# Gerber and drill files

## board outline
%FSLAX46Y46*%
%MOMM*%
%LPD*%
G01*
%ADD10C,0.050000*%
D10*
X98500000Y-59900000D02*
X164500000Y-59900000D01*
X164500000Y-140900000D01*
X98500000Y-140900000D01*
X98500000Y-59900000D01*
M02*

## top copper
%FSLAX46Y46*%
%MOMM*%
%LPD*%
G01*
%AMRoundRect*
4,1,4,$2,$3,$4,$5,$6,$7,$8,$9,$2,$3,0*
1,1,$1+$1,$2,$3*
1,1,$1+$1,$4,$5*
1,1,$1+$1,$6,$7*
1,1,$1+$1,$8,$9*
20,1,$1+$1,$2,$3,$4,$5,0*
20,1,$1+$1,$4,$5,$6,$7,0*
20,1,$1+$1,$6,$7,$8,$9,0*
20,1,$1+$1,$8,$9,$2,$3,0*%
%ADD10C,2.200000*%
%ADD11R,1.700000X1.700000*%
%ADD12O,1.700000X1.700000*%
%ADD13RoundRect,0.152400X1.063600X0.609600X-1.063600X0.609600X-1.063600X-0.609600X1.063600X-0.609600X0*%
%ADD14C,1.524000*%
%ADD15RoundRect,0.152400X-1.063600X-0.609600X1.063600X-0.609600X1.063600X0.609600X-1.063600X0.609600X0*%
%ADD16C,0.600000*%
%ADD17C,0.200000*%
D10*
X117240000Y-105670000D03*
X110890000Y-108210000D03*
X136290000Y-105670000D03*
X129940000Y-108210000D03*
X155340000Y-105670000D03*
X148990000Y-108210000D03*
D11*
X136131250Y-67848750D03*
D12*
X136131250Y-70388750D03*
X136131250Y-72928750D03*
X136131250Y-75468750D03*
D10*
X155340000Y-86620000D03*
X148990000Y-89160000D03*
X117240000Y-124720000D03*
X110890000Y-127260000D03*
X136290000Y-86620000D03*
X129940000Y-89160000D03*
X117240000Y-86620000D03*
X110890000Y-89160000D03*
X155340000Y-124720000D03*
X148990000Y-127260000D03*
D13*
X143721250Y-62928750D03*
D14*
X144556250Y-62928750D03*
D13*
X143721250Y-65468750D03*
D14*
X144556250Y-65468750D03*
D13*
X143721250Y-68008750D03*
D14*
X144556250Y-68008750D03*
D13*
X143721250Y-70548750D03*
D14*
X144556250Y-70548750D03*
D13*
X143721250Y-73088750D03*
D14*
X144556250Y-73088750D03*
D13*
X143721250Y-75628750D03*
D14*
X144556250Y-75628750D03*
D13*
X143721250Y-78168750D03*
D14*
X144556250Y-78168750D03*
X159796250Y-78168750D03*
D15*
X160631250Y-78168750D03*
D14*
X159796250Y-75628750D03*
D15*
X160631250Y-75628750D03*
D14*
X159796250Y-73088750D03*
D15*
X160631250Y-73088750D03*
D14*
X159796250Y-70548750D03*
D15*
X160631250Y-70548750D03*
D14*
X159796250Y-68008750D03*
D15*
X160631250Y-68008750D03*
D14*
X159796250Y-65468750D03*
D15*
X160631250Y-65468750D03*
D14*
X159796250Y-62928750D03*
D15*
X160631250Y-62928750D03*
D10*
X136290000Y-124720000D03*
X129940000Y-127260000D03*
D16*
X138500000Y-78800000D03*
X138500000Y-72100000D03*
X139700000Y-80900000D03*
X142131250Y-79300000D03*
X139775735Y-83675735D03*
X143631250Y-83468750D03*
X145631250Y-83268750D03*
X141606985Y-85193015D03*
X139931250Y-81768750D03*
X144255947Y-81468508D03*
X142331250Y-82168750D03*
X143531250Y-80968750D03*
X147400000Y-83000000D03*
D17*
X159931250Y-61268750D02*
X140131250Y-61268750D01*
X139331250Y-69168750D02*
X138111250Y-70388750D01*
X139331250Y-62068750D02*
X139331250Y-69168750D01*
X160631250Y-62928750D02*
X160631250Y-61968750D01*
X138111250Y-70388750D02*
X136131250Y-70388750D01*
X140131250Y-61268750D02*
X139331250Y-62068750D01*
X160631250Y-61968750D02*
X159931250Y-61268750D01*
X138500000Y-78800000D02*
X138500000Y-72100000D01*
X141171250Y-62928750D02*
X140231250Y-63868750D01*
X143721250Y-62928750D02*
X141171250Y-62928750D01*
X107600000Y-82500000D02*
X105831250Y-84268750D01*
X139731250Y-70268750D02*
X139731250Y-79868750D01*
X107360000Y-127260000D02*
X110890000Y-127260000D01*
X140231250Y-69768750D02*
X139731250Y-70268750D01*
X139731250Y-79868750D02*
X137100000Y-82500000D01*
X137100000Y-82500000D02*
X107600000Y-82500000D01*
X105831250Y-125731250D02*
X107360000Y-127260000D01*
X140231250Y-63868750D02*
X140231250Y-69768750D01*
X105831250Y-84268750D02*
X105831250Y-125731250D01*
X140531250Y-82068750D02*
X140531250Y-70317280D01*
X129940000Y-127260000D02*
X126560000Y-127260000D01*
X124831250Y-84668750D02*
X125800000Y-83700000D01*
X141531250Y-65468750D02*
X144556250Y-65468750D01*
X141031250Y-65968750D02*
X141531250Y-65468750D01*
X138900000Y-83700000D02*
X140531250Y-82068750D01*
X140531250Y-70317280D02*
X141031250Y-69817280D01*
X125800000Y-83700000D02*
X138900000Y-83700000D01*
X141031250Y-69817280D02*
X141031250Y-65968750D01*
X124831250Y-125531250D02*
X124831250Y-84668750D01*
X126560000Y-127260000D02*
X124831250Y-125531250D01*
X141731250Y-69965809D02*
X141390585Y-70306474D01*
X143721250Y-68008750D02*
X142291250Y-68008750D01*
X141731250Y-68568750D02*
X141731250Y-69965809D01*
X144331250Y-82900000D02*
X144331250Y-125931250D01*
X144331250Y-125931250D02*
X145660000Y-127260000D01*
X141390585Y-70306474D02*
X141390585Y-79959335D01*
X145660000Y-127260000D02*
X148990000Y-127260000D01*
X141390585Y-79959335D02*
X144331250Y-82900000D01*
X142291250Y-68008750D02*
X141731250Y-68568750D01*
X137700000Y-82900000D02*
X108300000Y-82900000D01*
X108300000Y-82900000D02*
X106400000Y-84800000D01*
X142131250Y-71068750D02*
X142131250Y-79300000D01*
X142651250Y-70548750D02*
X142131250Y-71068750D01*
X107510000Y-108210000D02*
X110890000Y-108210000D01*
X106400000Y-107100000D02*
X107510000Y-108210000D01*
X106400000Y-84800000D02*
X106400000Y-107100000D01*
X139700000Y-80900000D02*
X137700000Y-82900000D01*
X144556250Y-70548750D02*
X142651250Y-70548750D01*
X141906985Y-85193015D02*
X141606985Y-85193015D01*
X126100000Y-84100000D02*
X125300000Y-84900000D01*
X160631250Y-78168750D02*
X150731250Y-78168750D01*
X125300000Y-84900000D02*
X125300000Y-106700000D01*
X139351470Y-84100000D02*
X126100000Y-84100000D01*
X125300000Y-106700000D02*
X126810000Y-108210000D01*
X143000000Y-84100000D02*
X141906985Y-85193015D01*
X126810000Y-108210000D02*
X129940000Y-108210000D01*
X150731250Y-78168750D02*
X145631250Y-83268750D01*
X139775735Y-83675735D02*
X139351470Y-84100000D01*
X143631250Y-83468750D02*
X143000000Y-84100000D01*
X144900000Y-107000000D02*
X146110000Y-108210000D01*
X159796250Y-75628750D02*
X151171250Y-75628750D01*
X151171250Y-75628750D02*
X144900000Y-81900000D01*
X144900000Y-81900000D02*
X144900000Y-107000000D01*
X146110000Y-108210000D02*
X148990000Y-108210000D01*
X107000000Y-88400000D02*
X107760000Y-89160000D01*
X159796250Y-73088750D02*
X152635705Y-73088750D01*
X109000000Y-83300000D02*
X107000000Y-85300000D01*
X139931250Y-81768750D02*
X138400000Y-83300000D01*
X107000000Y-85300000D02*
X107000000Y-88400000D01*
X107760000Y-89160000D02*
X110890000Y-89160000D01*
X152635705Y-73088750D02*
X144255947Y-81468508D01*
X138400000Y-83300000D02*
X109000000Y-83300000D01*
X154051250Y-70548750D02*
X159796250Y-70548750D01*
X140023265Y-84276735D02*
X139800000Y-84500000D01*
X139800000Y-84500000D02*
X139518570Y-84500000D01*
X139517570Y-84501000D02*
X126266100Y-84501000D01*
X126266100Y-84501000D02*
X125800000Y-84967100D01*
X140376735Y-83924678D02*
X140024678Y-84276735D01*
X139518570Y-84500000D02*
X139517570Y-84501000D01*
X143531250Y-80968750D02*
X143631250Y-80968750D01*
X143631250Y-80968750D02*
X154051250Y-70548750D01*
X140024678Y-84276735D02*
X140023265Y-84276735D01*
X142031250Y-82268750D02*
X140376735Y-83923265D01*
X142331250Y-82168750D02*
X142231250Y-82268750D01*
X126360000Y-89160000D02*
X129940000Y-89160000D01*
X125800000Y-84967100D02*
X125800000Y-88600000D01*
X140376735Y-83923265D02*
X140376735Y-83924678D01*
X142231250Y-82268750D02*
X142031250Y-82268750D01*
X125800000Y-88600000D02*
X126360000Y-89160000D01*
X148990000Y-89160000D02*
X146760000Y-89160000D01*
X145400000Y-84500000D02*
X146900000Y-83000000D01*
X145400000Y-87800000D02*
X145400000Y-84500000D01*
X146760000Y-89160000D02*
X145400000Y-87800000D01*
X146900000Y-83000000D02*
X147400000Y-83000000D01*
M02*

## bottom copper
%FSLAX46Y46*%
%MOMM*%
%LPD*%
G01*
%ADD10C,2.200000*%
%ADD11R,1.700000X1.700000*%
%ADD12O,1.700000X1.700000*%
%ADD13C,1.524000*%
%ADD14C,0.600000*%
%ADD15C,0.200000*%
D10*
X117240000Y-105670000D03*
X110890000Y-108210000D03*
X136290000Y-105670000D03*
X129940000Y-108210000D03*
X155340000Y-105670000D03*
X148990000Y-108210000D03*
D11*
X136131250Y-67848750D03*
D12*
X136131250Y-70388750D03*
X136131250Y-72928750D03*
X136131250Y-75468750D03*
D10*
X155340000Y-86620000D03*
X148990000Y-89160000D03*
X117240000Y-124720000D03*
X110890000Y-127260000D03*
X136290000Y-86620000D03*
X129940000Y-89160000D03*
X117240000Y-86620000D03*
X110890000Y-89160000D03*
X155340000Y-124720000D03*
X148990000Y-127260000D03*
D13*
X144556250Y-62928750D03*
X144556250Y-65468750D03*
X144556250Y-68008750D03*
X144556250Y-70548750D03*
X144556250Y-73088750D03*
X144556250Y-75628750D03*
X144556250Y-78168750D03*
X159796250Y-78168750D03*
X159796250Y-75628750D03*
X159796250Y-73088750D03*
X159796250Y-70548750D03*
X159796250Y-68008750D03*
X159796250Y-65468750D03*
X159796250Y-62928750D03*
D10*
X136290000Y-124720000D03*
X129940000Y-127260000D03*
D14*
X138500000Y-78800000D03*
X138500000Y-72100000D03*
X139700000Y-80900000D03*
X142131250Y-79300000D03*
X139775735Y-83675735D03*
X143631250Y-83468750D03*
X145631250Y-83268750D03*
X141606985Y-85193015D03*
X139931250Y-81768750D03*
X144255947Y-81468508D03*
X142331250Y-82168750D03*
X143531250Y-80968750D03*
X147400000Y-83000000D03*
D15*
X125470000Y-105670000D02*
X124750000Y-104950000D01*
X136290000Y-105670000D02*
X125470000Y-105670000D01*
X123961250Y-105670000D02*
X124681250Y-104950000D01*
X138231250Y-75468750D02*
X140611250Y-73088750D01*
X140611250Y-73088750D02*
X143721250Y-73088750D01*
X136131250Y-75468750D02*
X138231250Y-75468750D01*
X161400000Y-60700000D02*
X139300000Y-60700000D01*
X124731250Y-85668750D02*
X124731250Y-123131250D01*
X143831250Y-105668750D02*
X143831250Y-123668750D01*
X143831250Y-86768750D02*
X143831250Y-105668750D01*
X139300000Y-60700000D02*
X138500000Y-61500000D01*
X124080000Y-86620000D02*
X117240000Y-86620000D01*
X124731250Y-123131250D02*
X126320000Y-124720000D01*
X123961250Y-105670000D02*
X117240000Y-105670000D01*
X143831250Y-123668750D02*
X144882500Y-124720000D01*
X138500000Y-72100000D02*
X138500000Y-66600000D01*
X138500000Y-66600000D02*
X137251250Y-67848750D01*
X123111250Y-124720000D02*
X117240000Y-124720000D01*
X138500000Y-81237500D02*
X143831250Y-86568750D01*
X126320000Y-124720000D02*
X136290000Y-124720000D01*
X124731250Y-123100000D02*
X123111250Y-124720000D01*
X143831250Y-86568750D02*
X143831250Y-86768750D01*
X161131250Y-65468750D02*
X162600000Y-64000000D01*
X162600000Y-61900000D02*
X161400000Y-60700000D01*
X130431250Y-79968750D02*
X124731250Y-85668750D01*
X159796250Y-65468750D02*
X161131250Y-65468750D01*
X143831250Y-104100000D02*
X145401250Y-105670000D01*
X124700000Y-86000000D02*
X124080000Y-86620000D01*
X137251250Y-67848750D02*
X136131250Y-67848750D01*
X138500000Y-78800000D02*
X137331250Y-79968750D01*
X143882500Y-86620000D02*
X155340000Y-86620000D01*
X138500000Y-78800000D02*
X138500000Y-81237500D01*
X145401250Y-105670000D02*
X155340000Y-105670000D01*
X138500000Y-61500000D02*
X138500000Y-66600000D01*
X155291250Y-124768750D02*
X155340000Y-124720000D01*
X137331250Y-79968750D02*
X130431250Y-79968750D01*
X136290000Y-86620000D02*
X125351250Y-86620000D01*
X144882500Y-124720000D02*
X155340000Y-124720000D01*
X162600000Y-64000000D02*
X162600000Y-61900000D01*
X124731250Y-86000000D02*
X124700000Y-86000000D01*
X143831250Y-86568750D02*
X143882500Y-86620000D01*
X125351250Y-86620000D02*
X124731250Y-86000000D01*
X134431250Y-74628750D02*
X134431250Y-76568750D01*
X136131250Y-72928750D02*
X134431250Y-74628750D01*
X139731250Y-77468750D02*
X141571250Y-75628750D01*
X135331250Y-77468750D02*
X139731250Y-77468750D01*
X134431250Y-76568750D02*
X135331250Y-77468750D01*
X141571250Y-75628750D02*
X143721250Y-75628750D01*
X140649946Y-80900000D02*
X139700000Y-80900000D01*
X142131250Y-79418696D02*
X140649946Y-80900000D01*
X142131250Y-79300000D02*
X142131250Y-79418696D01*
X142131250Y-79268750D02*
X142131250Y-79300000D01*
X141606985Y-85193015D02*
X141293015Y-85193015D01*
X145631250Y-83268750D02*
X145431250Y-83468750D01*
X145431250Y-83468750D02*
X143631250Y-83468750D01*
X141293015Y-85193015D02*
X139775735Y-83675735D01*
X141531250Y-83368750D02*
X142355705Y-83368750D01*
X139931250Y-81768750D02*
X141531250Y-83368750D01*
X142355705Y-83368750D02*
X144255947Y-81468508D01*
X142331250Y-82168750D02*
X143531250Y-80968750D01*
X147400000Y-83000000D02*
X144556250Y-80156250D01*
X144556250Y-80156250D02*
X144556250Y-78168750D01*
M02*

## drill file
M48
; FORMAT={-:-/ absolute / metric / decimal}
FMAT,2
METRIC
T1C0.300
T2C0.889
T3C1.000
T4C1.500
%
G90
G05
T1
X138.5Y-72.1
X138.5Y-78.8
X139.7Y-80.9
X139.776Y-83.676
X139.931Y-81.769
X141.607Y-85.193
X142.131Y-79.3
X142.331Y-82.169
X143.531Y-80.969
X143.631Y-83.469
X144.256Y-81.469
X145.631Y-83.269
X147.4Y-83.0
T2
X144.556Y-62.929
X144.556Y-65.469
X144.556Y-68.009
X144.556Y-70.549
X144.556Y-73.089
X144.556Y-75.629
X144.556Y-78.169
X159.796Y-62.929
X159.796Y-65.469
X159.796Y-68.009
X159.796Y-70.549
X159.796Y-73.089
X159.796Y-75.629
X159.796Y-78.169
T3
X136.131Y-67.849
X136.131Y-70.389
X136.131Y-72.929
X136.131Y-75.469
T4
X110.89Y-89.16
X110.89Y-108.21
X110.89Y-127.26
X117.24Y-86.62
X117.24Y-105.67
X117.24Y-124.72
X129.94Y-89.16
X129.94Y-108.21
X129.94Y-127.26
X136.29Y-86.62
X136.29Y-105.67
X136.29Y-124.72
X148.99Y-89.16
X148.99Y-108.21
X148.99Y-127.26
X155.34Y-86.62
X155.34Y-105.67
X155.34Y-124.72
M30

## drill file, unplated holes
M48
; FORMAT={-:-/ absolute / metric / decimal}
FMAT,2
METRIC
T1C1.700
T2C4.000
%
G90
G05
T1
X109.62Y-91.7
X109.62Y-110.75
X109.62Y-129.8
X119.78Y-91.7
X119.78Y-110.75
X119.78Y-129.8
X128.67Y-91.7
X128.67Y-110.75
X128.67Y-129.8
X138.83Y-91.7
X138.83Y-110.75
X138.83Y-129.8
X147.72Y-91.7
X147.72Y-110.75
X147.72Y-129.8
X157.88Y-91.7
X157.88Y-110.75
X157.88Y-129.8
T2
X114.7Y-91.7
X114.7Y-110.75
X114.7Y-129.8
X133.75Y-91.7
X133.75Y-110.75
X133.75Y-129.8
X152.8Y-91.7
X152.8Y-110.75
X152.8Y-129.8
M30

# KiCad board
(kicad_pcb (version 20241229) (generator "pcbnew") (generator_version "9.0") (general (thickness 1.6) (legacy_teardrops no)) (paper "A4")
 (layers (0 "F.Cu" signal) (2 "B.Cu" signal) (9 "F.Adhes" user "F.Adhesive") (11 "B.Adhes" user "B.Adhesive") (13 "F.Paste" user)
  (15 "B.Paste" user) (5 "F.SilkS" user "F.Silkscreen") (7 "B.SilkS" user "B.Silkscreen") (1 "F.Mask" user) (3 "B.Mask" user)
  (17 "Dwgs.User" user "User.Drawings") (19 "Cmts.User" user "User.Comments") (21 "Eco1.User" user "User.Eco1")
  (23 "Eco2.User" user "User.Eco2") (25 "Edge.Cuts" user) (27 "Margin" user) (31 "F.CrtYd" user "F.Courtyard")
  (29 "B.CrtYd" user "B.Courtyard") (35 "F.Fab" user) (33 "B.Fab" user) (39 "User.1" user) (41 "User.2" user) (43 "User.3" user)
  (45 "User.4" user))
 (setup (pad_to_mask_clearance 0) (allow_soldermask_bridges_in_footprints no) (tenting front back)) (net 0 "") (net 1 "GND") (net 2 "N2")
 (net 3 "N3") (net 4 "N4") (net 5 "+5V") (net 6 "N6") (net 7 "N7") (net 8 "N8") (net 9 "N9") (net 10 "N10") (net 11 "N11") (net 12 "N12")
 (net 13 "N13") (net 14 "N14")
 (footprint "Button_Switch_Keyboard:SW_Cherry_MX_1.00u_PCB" (layer "F.Cu") (at 117.24 105.67)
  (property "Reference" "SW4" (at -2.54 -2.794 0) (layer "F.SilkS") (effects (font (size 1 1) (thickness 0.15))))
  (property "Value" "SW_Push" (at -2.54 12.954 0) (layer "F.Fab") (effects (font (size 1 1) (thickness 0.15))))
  (pad "" np_thru_hole circle (at -7.62 5.08) (size 1.7 1.7) (drill 1.7) (layers "*.Cu" "*.Mask"))
  (pad "" np_thru_hole circle (at -2.54 5.08) (size 4 4) (drill 4) (layers "*.Cu" "*.Mask"))
  (pad "" np_thru_hole circle (at 2.54 5.08) (size 1.7 1.7) (drill 1.7) (layers "*.Cu" "*.Mask"))
  (pad "1" thru_hole circle (at 0 0) (size 2.2 2.2) (drill 1.5) (layers "*.Cu" "*.Mask") (remove_unused_layers no) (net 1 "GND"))
  (pad "2" thru_hole circle (at -6.35 2.54) (size 2.2 2.2) (drill 1.5) (layers "*.Cu" "*.Mask") (remove_unused_layers no) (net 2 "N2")))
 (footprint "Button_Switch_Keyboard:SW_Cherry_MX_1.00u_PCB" (layer "F.Cu") (at 136.29 105.67)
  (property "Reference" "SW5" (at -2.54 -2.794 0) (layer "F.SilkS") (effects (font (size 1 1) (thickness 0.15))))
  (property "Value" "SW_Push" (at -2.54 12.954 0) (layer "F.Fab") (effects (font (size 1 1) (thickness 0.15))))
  (pad "" np_thru_hole circle (at -7.62 5.08) (size 1.7 1.7) (drill 1.7) (layers "*.Cu" "*.Mask"))
  (pad "" np_thru_hole circle (at -2.54 5.08) (size 4 4) (drill 4) (layers "*.Cu" "*.Mask"))
  (pad "" np_thru_hole circle (at 2.54 5.08) (size 1.7 1.7) (drill 1.7) (layers "*.Cu" "*.Mask"))
  (pad "1" thru_hole circle (at 0 0) (size 2.2 2.2) (drill 1.5) (layers "*.Cu" "*.Mask") (remove_unused_layers no) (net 1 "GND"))
  (pad "2" thru_hole circle (at -6.35 2.54) (size 2.2 2.2) (drill 1.5) (layers "*.Cu" "*.Mask") (remove_unused_layers no) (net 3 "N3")))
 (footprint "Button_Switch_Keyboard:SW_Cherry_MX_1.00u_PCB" (layer "F.Cu") (at 155.34 105.67)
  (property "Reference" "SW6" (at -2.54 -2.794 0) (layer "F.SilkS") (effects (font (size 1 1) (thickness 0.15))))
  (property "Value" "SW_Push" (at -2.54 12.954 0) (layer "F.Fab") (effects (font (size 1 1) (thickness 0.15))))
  (pad "" np_thru_hole circle (at -7.62 5.08) (size 1.7 1.7) (drill 1.7) (layers "*.Cu" "*.Mask"))
  (pad "" np_thru_hole circle (at -2.54 5.08) (size 4 4) (drill 4) (layers "*.Cu" "*.Mask"))
  (pad "" np_thru_hole circle (at 2.54 5.08) (size 1.7 1.7) (drill 1.7) (layers "*.Cu" "*.Mask"))
  (pad "1" thru_hole circle (at 0 0) (size 2.2 2.2) (drill 1.5) (layers "*.Cu" "*.Mask") (remove_unused_layers no) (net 1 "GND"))
  (pad "2" thru_hole circle (at -6.35 2.54) (size 2.2 2.2) (drill 1.5) (layers "*.Cu" "*.Mask") (remove_unused_layers no) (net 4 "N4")))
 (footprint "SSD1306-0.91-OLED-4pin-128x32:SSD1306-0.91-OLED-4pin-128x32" (layer "F.Cu") (at 99.63125 65.65875)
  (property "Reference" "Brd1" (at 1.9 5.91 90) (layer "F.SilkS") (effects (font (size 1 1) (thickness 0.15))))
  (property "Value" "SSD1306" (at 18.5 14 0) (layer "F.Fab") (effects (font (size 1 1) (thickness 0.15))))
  (pad "1" thru_hole rect (at 36.5 2.19) (size 1.7 1.7) (drill 1) (layers "*.Cu" "*.Mask") (remove_unused_layers no) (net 1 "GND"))
  (pad "2" thru_hole oval (at 36.5 4.73) (size 1.7 1.7) (drill 1) (layers "*.Cu" "*.Mask") (remove_unused_layers no) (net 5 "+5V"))
  (pad "3" thru_hole oval (at 36.5 7.27) (size 1.7 1.7) (drill 1) (layers "*.Cu" "*.Mask") (remove_unused_layers no) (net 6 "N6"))
  (pad "4" thru_hole oval (at 36.5 9.81) (size 1.7 1.7) (drill 1) (layers "*.Cu" "*.Mask") (remove_unused_layers no) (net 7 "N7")))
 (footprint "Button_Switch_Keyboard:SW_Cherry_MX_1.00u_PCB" (layer "F.Cu") (at 155.34 86.62)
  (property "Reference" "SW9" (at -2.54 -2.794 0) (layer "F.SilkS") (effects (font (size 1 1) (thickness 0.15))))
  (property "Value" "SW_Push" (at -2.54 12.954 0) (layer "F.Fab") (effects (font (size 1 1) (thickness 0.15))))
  (pad "" np_thru_hole circle (at -7.62 5.08) (size 1.7 1.7) (drill 1.7) (layers "*.Cu" "*.Mask"))
  (pad "" np_thru_hole circle (at -2.54 5.08) (size 4 4) (drill 4) (layers "*.Cu" "*.Mask"))
  (pad "" np_thru_hole circle (at 2.54 5.08) (size 1.7 1.7) (drill 1.7) (layers "*.Cu" "*.Mask"))
  (pad "1" thru_hole circle (at 0 0) (size 2.2 2.2) (drill 1.5) (layers "*.Cu" "*.Mask") (remove_unused_layers no) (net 1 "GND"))
  (pad "2" thru_hole circle (at -6.35 2.54) (size 2.2 2.2) (drill 1.5) (layers "*.Cu" "*.Mask") (remove_unused_layers no) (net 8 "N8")))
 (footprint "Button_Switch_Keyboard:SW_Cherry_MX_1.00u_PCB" (layer "F.Cu") (at 117.24 124.72)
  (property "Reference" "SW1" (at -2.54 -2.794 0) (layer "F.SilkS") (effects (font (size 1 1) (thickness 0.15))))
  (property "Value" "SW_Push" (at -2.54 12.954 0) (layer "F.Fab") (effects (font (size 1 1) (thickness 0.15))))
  (pad "" np_thru_hole circle (at -7.62 5.08) (size 1.7 1.7) (drill 1.7) (layers "*.Cu" "*.Mask"))
  (pad "" np_thru_hole circle (at -2.54 5.08) (size 4 4) (drill 4) (layers "*.Cu" "*.Mask"))
  (pad "" np_thru_hole circle (at 2.54 5.08) (size 1.7 1.7) (drill 1.7) (layers "*.Cu" "*.Mask"))
  (pad "1" thru_hole circle (at 0 0) (size 2.2 2.2) (drill 1.5) (layers "*.Cu" "*.Mask") (remove_unused_layers no) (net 1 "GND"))
  (pad "2" thru_hole circle (at -6.35 2.54) (size 2.2 2.2) (drill 1.5) (layers "*.Cu" "*.Mask") (remove_unused_layers no) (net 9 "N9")))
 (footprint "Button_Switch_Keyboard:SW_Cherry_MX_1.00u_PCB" (layer "F.Cu") (at 136.29 86.62)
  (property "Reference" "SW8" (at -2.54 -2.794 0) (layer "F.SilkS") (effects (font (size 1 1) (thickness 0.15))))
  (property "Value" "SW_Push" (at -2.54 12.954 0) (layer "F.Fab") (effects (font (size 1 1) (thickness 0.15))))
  (pad "" np_thru_hole circle (at -7.62 5.08) (size 1.7 1.7) (drill 1.7) (layers "*.Cu" "*.Mask"))
  (pad "" np_thru_hole circle (at -2.54 5.08) (size 4 4) (drill 4) (layers "*.Cu" "*.Mask"))
  (pad "" np_thru_hole circle (at 2.54 5.08) (size 1.7 1.7) (drill 1.7) (layers "*.Cu" "*.Mask"))
  (pad "1" thru_hole circle (at 0 0) (size 2.2 2.2) (drill 1.5) (layers "*.Cu" "*.Mask") (remove_unused_layers no) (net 1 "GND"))
  (pad "2" thru_hole circle (at -6.35 2.54) (size 2.2 2.2) (drill 1.5) (layers "*.Cu" "*.Mask") (remove_unused_layers no) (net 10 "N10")))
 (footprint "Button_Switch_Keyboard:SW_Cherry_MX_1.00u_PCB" (layer "F.Cu") (at 117.24 86.62)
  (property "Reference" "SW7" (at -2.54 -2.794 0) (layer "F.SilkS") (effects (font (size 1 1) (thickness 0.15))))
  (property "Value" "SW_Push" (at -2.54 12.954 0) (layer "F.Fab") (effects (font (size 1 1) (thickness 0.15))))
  (pad "" np_thru_hole circle (at -7.62 5.08) (size 1.7 1.7) (drill 1.7) (layers "*.Cu" "*.Mask"))
  (pad "" np_thru_hole circle (at -2.54 5.08) (size 4 4) (drill 4) (layers "*.Cu" "*.Mask"))
  (pad "" np_thru_hole circle (at 2.54 5.08) (size 1.7 1.7) (drill 1.7) (layers "*.Cu" "*.Mask"))
  (pad "1" thru_hole circle (at 0 0) (size 2.2 2.2) (drill 1.5) (layers "*.Cu" "*.Mask") (remove_unused_layers no) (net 1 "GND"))
  (pad "2" thru_hole circle (at -6.35 2.54) (size 2.2 2.2) (drill 1.5) (layers "*.Cu" "*.Mask") (remove_unused_layers no) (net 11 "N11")))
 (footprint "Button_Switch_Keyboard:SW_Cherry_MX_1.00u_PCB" (layer "F.Cu") (at 155.34 124.72)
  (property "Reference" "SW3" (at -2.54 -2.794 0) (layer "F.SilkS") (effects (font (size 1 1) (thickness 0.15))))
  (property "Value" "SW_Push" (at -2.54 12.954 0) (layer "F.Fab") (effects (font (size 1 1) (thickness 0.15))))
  (pad "" np_thru_hole circle (at -7.62 5.08) (size 1.7 1.7) (drill 1.7) (layers "*.Cu" "*.Mask"))
  (pad "" np_thru_hole circle (at -2.54 5.08) (size 4 4) (drill 4) (layers "*.Cu" "*.Mask"))
  (pad "" np_thru_hole circle (at 2.54 5.08) (size 1.7 1.7) (drill 1.7) (layers "*.Cu" "*.Mask"))
  (pad "1" thru_hole circle (at 0 0) (size 2.2 2.2) (drill 1.5) (layers "*.Cu" "*.Mask") (remove_unused_layers no) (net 1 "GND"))
  (pad "2" thru_hole circle (at -6.35 2.54) (size 2.2 2.2) (drill 1.5) (layers "*.Cu" "*.Mask") (remove_unused_layers no) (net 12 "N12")))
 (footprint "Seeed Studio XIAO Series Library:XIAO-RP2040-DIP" (layer "F.Cu") (at 152.17625 70.54875)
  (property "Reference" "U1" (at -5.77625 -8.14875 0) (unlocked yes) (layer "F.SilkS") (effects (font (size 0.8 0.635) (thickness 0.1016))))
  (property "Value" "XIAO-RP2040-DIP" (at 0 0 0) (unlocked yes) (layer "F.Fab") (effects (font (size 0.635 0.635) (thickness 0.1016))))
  (pad "1" smd roundrect (at -8.455 -7.62 180) (size 2.432 1.524) (layers "F.Cu" "F.Mask") (roundrect_rratio 0.1) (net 9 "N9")
   (thermal_bridge_angle 45))
  (pad "1" thru_hole circle (at -7.62 -7.62 180) (size 1.524 1.524) (drill 0.889) (layers "*.Cu" "*.Mask") (remove_unused_layers no)
   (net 9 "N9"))
  (pad "2" smd roundrect (at -8.455 -5.08 180) (size 2.432 1.524) (layers "F.Cu" "F.Mask") (roundrect_rratio 0.1) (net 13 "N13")
   (thermal_bridge_angle 45))
  (pad "2" thru_hole circle (at -7.62 -5.08 180) (size 1.524 1.524) (drill 0.889) (layers "*.Cu" "*.Mask") (remove_unused_layers no)
   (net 13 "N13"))
  (pad "3" smd roundrect (at -8.455 -2.54 180) (size 2.432 1.524) (layers "F.Cu" "F.Mask") (roundrect_rratio 0.1) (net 12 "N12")
   (thermal_bridge_angle 45))
  (pad "3" thru_hole circle (at -7.62 -2.54 180) (size 1.524 1.524) (drill 0.889) (layers "*.Cu" "*.Mask") (remove_unused_layers no)
   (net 12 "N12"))
  (pad "4" smd roundrect (at -8.455 0 180) (size 2.432 1.524) (layers "F.Cu" "F.Mask") (roundrect_rratio 0.1) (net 2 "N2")
   (thermal_bridge_angle 45))
  (pad "4" thru_hole circle (at -7.62 0 180) (size 1.524 1.524) (drill 0.889) (layers "*.Cu" "*.Mask") (remove_unused_layers no)
   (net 2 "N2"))
  (pad "5" smd roundrect (at -8.455 2.54 180) (size 2.432 1.524) (layers "F.Cu" "F.Mask") (roundrect_rratio 0.1) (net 7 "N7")
   (thermal_bridge_angle 45))
  (pad "5" thru_hole circle (at -7.62 2.54 180) (size 1.524 1.524) (drill 0.889) (layers "*.Cu" "*.Mask") (remove_unused_layers no)
   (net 7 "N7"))
  (pad "6" smd roundrect (at -8.455 5.08 180) (size 2.432 1.524) (layers "F.Cu" "F.Mask") (roundrect_rratio 0.1) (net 6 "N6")
   (thermal_bridge_angle 45))
  (pad "6" thru_hole circle (at -7.62 5.08 180) (size 1.524 1.524) (drill 0.889) (layers "*.Cu" "*.Mask") (remove_unused_layers no)
   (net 6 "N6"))
  (pad "7" smd roundrect (at -8.455 7.62 180) (size 2.432 1.524) (layers "F.Cu" "F.Mask") (roundrect_rratio 0.1) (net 8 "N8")
   (thermal_bridge_angle 45))
  (pad "7" thru_hole circle (at -7.62 7.62 180) (size 1.524 1.524) (drill 0.889) (layers "*.Cu" "*.Mask") (remove_unused_layers no)
   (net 8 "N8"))
  (pad "8" thru_hole circle (at 7.62 7.62) (size 1.524 1.524) (drill 0.889) (layers "*.Cu" "*.Mask") (remove_unused_layers no) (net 3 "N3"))
  (pad "8" smd roundrect (at 8.455 7.62) (size 2.432 1.524) (layers "F.Cu" "F.Mask") (roundrect_rratio 0.1) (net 3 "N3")
   (thermal_bridge_angle 45))
  (pad "9" thru_hole circle (at 7.62 5.08) (size 1.524 1.524) (drill 0.889) (layers "*.Cu" "*.Mask") (remove_unused_layers no) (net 4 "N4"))
  (pad "9" smd roundrect (at 8.455 5.08) (size 2.432 1.524) (layers "F.Cu" "F.Mask") (roundrect_rratio 0.1) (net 4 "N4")
   (thermal_bridge_angle 45))
  (pad "10" thru_hole circle (at 7.62 2.54) (size 1.524 1.524) (drill 0.889) (layers "*.Cu" "*.Mask") (remove_unused_layers no)
   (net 11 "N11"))
  (pad "10" smd roundrect (at 8.455 2.54) (size 2.432 1.524) (layers "F.Cu" "F.Mask") (roundrect_rratio 0.1) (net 11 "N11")
   (thermal_bridge_angle 45))
  (pad "11" thru_hole circle (at 7.62 0) (size 1.524 1.524) (drill 0.889) (layers "*.Cu" "*.Mask") (remove_unused_layers no) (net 10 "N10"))
  (pad "11" smd roundrect (at 8.455 0) (size 2.432 1.524) (layers "F.Cu" "F.Mask") (roundrect_rratio 0.1) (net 10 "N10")
   (thermal_bridge_angle 45))
  (pad "12" thru_hole circle (at 7.62 -2.54) (size 1.524 1.524) (drill 0.889) (layers "*.Cu" "*.Mask") (remove_unused_layers no)
   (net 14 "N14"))
  (pad "12" smd roundrect (at 8.455 -2.54) (size 2.432 1.524) (layers "F.Cu" "F.Mask") (roundrect_rratio 0.1) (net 14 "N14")
   (thermal_bridge_angle 45))
  (pad "13" thru_hole circle (at 7.62 -5.08) (size 1.524 1.524) (drill 0.889) (layers "*.Cu" "*.Mask") (remove_unused_layers no)
   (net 1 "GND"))
  (pad "13" smd roundrect (at 8.455 -5.08) (size 2.432 1.524) (layers "F.Cu" "F.Mask") (roundrect_rratio 0.1) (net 1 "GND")
   (thermal_bridge_angle 45))
  (pad "14" thru_hole circle (at 7.62 -7.62) (size 1.524 1.524) (drill 0.889) (layers "*.Cu" "*.Mask") (remove_unused_layers no)
   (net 5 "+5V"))
  (pad "14" smd roundrect (at 8.455 -7.62) (size 2.432 1.524) (layers "F.Cu" "F.Mask") (roundrect_rratio 0.1) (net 5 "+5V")
   (thermal_bridge_angle 45)))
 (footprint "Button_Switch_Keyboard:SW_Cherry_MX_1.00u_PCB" (layer "F.Cu") (at 136.29 124.72)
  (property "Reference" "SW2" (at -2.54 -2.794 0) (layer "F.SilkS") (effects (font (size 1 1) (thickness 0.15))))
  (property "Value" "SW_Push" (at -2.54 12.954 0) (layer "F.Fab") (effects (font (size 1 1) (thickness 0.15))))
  (pad "" np_thru_hole circle (at -7.62 5.08) (size 1.7 1.7) (drill 1.7) (layers "*.Cu" "*.Mask"))
  (pad "" np_thru_hole circle (at -2.54 5.08) (size 4 4) (drill 4) (layers "*.Cu" "*.Mask"))
  (pad "" np_thru_hole circle (at 2.54 5.08) (size 1.7 1.7) (drill 1.7) (layers "*.Cu" "*.Mask"))
  (pad "1" thru_hole circle (at 0 0) (size 2.2 2.2) (drill 1.5) (layers "*.Cu" "*.Mask") (remove_unused_layers no) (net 1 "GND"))
  (pad "2" thru_hole circle (at -6.35 2.54) (size 2.2 2.2) (drill 1.5) (layers "*.Cu" "*.Mask") (remove_unused_layers no) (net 13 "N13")))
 (gr_rect (start 98.5 59.9) (end 164.5 140.9) (stroke (width 0.05) (type solid)) (fill no) (layer "Edge.Cuts"))
 (segment (start 138.23125 75.46875) (end 140.61125 73.08875) (width 0.2) (layer "B.Cu") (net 7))
 (segment (start 140.61125 73.08875) (end 143.72125 73.08875) (width 0.2) (layer "B.Cu") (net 7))
 (segment (start 136.13125 75.46875) (end 138.23125 75.46875) (width 0.2) (layer "B.Cu") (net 7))
 (segment (start 159.93125 61.26875) (end 140.13125 61.26875) (width 0.2) (layer "F.Cu") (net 5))
 (segment (start 139.33125 69.16875) (end 138.11125 70.38875) (width 0.2) (layer "F.Cu") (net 5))
 (segment (start 139.33125 62.06875) (end 139.33125 69.16875) (width 0.2) (layer "F.Cu") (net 5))
 (segment (start 160.63125 62.92875) (end 160.63125 61.96875) (width 0.2) (layer "F.Cu") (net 5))
 (segment (start 138.11125 70.38875) (end 136.13125 70.38875) (width 0.2) (layer "F.Cu") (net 5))
 (segment (start 140.13125 61.26875) (end 139.33125 62.06875) (width 0.2) (layer "F.Cu") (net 5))
 (segment (start 160.63125 61.96875) (end 159.93125 61.26875) (width 0.2) (layer "F.Cu") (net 5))
 (segment (start 138.5 78.8) (end 138.5 72.1) (width 0.2) (layer "F.Cu") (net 1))
 (via (at 138.5 78.8) (size 0.6) (drill 0.3) (layers "F.Cu" "B.Cu") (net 1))
 (via (at 138.5 72.1) (size 0.6) (drill 0.3) (layers "F.Cu" "B.Cu") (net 1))
 (segment (start 161.4 60.7) (end 139.3 60.7) (width 0.2) (layer "B.Cu") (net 1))
 (segment (start 124.73125 85.66875) (end 124.73125 123.13125) (width 0.2) (layer "B.Cu") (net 1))
 (segment (start 143.83125 105.66875) (end 143.83125 123.66875) (width 0.2) (layer "B.Cu") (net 1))
 (segment (start 143.83125 86.76875) (end 143.83125 105.66875) (width 0.2) (layer "B.Cu") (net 1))
 (segment (start 139.3 60.7) (end 138.5 61.5) (width 0.2) (layer "B.Cu") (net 1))
 (segment (start 124.08 86.62) (end 117.24 86.62) (width 0.2) (layer "B.Cu") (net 1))
 (segment (start 124.73125 123.13125) (end 126.32 124.72) (width 0.2) (layer "B.Cu") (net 1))
 (segment (start 123.96125 105.67) (end 117.24 105.67) (width 0.2) (layer "B.Cu") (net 1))
 (segment (start 143.83125 123.66875) (end 144.8825 124.72) (width 0.2) (layer "B.Cu") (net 1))
 (segment (start 138.5 72.1) (end 138.5 66.6) (width 0.2) (layer "B.Cu") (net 1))
 (segment (start 138.5 66.6) (end 137.25125 67.84875) (width 0.2) (layer "B.Cu") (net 1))
 (segment (start 123.11125 124.72) (end 117.24 124.72) (width 0.2) (layer "B.Cu") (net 1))
 (segment (start 138.5 81.2375) (end 143.83125 86.56875) (width 0.2) (layer "B.Cu") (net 1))
 (segment (start 126.32 124.72) (end 136.29 124.72) (width 0.2) (layer "B.Cu") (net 1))
 (segment (start 124.73125 123.1) (end 123.11125 124.72) (width 0.2) (layer "B.Cu") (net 1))
 (segment (start 143.83125 86.56875) (end 143.83125 86.76875) (width 0.2) (layer "B.Cu") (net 1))
 (segment (start 161.13125 65.46875) (end 162.6 64) (width 0.2) (layer "B.Cu") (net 1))
 (segment (start 162.6 61.9) (end 161.4 60.7) (width 0.2) (layer "B.Cu") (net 1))
 (segment (start 130.43125 79.96875) (end 124.73125 85.66875) (width 0.2) (layer "B.Cu") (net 1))
 (segment (start 159.79625 65.46875) (end 161.13125 65.46875) (width 0.2) (layer "B.Cu") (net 1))
 (segment (start 143.83125 104.1) (end 145.40125 105.67) (width 0.2) (layer "B.Cu") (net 1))
 (segment (start 124.7 86) (end 124.08 86.62) (width 0.2) (layer "B.Cu") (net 1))
 (segment (start 125.47 105.67) (end 124.75 104.95) (width 0.2) (layer "B.Cu") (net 1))
 (segment (start 137.25125 67.84875) (end 136.13125 67.84875) (width 0.2) (layer "B.Cu") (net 1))
 (segment (start 138.5 78.8) (end 137.33125 79.96875) (width 0.2) (layer "B.Cu") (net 1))
 (segment (start 143.8825 86.62) (end 155.34 86.62) (width 0.2) (layer "B.Cu") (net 1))
 (segment (start 138.5 78.8) (end 138.5 81.2375) (width 0.2) (layer "B.Cu") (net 1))
 (segment (start 145.40125 105.67) (end 155.34 105.67) (width 0.2) (layer "B.Cu") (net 1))
 (segment (start 138.5 61.5) (end 138.5 66.6) (width 0.2) (layer "B.Cu") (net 1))
 (segment (start 123.96125 105.67) (end 124.68125 104.95) (width 0.2) (layer "B.Cu") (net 1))
 (segment (start 155.29125 124.76875) (end 155.34 124.72) (width 0.2) (layer "B.Cu") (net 1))
 (segment (start 137.33125 79.96875) (end 130.43125 79.96875) (width 0.2) (layer "B.Cu") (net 1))
 (segment (start 136.29 105.67) (end 125.47 105.67) (width 0.2) (layer "B.Cu") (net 1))
 (segment (start 136.29 86.62) (end 125.35125 86.62) (width 0.2) (layer "B.Cu") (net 1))
 (segment (start 144.8825 124.72) (end 155.34 124.72) (width 0.2) (layer "B.Cu") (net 1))
 (segment (start 162.6 64) (end 162.6 61.9) (width 0.2) (layer "B.Cu") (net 1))
 (segment (start 124.73125 86) (end 124.7 86) (width 0.2) (layer "B.Cu") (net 1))
 (segment (start 143.83125 86.56875) (end 143.8825 86.62) (width 0.2) (layer "B.Cu") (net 1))
 (segment (start 125.35125 86.62) (end 124.73125 86) (width 0.2) (layer "B.Cu") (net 1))
 (segment (start 134.43125 74.62875) (end 134.43125 76.56875) (width 0.2) (layer "B.Cu") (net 6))
 (segment (start 136.13125 72.92875) (end 134.43125 74.62875) (width 0.2) (layer "B.Cu") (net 6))
 (segment (start 139.73125 77.46875) (end 141.57125 75.62875) (width 0.2) (layer "B.Cu") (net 6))
 (segment (start 135.33125 77.46875) (end 139.73125 77.46875) (width 0.2) (layer "B.Cu") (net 6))
 (segment (start 134.43125 76.56875) (end 135.33125 77.46875) (width 0.2) (layer "B.Cu") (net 6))
 (segment (start 141.57125 75.62875) (end 143.72125 75.62875) (width 0.2) (layer "B.Cu") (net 6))
 (segment (start 141.17125 62.92875) (end 140.23125 63.86875) (width 0.2) (layer "F.Cu") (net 9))
 (segment (start 143.72125 62.92875) (end 141.17125 62.92875) (width 0.2) (layer "F.Cu") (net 9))
 (segment (start 107.6 82.5) (end 105.83125 84.26875) (width 0.2) (layer "F.Cu") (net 9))
 (segment (start 139.73125 70.26875) (end 139.73125 79.86875) (width 0.2) (layer "F.Cu") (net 9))
 (segment (start 107.36 127.26) (end 110.89 127.26) (width 0.2) (layer "F.Cu") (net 9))
 (segment (start 140.23125 69.76875) (end 139.73125 70.26875) (width 0.2) (layer "F.Cu") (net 9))
 (segment (start 139.73125 79.86875) (end 137.1 82.5) (width 0.2) (layer "F.Cu") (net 9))
 (segment (start 137.1 82.5) (end 107.6 82.5) (width 0.2) (layer "F.Cu") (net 9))
 (segment (start 105.83125 125.73125) (end 107.36 127.26) (width 0.2) (layer "F.Cu") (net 9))
 (segment (start 140.23125 63.86875) (end 140.23125 69.76875) (width 0.2) (layer "F.Cu") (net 9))
 (segment (start 105.83125 84.26875) (end 105.83125 125.73125) (width 0.2) (layer "F.Cu") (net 9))
 (segment (start 140.53125 82.06875) (end 140.53125 70.31728) (width 0.2) (layer "F.Cu") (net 13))
 (segment (start 129.94 127.26) (end 126.56 127.26) (width 0.2) (layer "F.Cu") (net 13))
 (segment (start 124.83125 84.66875) (end 125.8 83.7) (width 0.2) (layer "F.Cu") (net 13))
 (segment (start 141.53125 65.46875) (end 144.55625 65.46875) (width 0.2) (layer "F.Cu") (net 13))
 (segment (start 141.03125 65.96875) (end 141.53125 65.46875) (width 0.2) (layer "F.Cu") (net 13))
 (segment (start 138.9 83.7) (end 140.53125 82.06875) (width 0.2) (layer "F.Cu") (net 13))
 (segment (start 140.53125 70.31728) (end 141.03125 69.81728) (width 0.2) (layer "F.Cu") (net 13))
 (segment (start 125.8 83.7) (end 138.9 83.7) (width 0.2) (layer "F.Cu") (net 13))
 (segment (start 141.03125 69.81728) (end 141.03125 65.96875) (width 0.2) (layer "F.Cu") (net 13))
 (segment (start 124.83125 125.53125) (end 124.83125 84.66875) (width 0.2) (layer "F.Cu") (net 13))
 (segment (start 126.56 127.26) (end 124.83125 125.53125) (width 0.2) (layer "F.Cu") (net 13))
 (segment (start 141.73125 69.965809) (end 141.390585 70.306474) (width 0.2) (layer "F.Cu") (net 12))
 (segment (start 143.72125 68.00875) (end 142.29125 68.00875) (width 0.2) (layer "F.Cu") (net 12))
 (segment (start 141.73125 68.56875) (end 141.73125 69.965809) (width 0.2) (layer "F.Cu") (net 12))
 (segment (start 144.33125 82.9) (end 144.33125 125.93125) (width 0.2) (layer "F.Cu") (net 12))
 (segment (start 144.33125 125.93125) (end 145.66 127.26) (width 0.2) (layer "F.Cu") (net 12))
 (segment (start 141.390585 70.306474) (end 141.390585 79.959335) (width 0.2) (layer "F.Cu") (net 12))
 (segment (start 145.66 127.26) (end 148.99 127.26) (width 0.2) (layer "F.Cu") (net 12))
 (segment (start 141.390585 79.959335) (end 144.33125 82.9) (width 0.2) (layer "F.Cu") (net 12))
 (segment (start 142.29125 68.00875) (end 141.73125 68.56875) (width 0.2) (layer "F.Cu") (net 12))
 (segment (start 137.7 82.9) (end 108.3 82.9) (width 0.2) (layer "F.Cu") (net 2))
 (segment (start 108.3 82.9) (end 106.4 84.8) (width 0.2) (layer "F.Cu") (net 2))
 (segment (start 142.13125 71.06875) (end 142.13125 79.3) (width 0.2) (layer "F.Cu") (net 2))
 (segment (start 142.65125 70.54875) (end 142.13125 71.06875) (width 0.2) (layer "F.Cu") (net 2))
 (segment (start 107.51 108.21) (end 110.89 108.21) (width 0.2) (layer "F.Cu") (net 2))
 (segment (start 106.4 107.1) (end 107.51 108.21) (width 0.2) (layer "F.Cu") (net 2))
 (segment (start 106.4 84.8) (end 106.4 107.1) (width 0.2) (layer "F.Cu") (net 2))
 (segment (start 139.7 80.9) (end 137.7 82.9) (width 0.2) (layer "F.Cu") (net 2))
 (segment (start 144.55625 70.54875) (end 142.65125 70.54875) (width 0.2) (layer "F.Cu") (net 2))
 (via (at 139.7 80.9) (size 0.6) (drill 0.3) (layers "F.Cu" "B.Cu") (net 2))
 (via (at 142.13125 79.3) (size 0.6) (drill 0.3) (layers "F.Cu" "B.Cu") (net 2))
 (segment (start 140.649946 80.9) (end 139.7 80.9) (width 0.2) (layer "B.Cu") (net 2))
 (segment (start 142.13125 79.418696) (end 140.649946 80.9) (width 0.2) (layer "B.Cu") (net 2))
 (segment (start 142.13125 79.3) (end 142.13125 79.418696) (width 0.2) (layer "B.Cu") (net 2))
 (segment (start 142.13125 79.26875) (end 142.13125 79.3) (width 0.2) (layer "B.Cu") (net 2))
 (segment (start 141.906985 85.193015) (end 141.606985 85.193015) (width 0.2) (layer "F.Cu") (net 3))
 (segment (start 126.1 84.1) (end 125.3 84.9) (width 0.2) (layer "F.Cu") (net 3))
 (segment (start 160.63125 78.16875) (end 150.73125 78.16875) (width 0.2) (layer "F.Cu") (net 3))
 (segment (start 125.3 84.9) (end 125.3 106.7) (width 0.2) (layer "F.Cu") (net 3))
 (segment (start 139.35147 84.1) (end 126.1 84.1) (width 0.2) (layer "F.Cu") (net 3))
 (segment (start 125.3 106.7) (end 126.81 108.21) (width 0.2) (layer "F.Cu") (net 3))
 (segment (start 143 84.1) (end 141.906985 85.193015) (width 0.2) (layer "F.Cu") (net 3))
 (segment (start 126.81 108.21) (end 129.94 108.21) (width 0.2) (layer "F.Cu") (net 3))
 (segment (start 150.73125 78.16875) (end 145.63125 83.26875) (width 0.2) (layer "F.Cu") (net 3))
 (segment (start 139.775735 83.675735) (end 139.35147 84.1) (width 0.2) (layer "F.Cu") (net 3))
 (segment (start 143.63125 83.46875) (end 143 84.1) (width 0.2) (layer "F.Cu") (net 3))
 (via (at 139.775735 83.675735) (size 0.6) (drill 0.3) (layers "F.Cu" "B.Cu") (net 3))
 (via (at 143.63125 83.46875) (size 0.6) (drill 0.3) (layers "F.Cu" "B.Cu") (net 3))
 (via (at 145.63125 83.26875) (size 0.6) (drill 0.3) (layers "F.Cu" "B.Cu") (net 3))
 (via (at 141.606985 85.193015) (size 0.6) (drill 0.3) (layers "F.Cu" "B.Cu") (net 3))
 (segment (start 141.606985 85.193015) (end 141.293015 85.193015) (width 0.2) (layer "B.Cu") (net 3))
 (segment (start 145.63125 83.26875) (end 145.43125 83.46875) (width 0.2) (layer "B.Cu") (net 3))
 (segment (start 145.43125 83.46875) (end 143.63125 83.46875) (width 0.2) (layer "B.Cu") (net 3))
 (segment (start 141.293015 85.193015) (end 139.775735 83.675735) (width 0.2) (layer "B.Cu") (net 3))
 (segment (start 144.9 107) (end 146.11 108.21) (width 0.2) (layer "F.Cu") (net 4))
 (segment (start 159.79625 75.62875) (end 151.17125 75.62875) (width 0.2) (layer "F.Cu") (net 4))
 (segment (start 151.17125 75.62875) (end 144.9 81.9) (width 0.2) (layer "F.Cu") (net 4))
 (segment (start 144.9 81.9) (end 144.9 107) (width 0.2) (layer "F.Cu") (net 4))
 (segment (start 146.11 108.21) (end 148.99 108.21) (width 0.2) (layer "F.Cu") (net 4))
 (segment (start 107 88.4) (end 107.76 89.16) (width 0.2) (layer "F.Cu") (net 11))
 (segment (start 159.79625 73.08875) (end 152.635705 73.08875) (width 0.2) (layer "F.Cu") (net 11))
 (segment (start 109 83.3) (end 107 85.3) (width 0.2) (layer "F.Cu") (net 11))
 (segment (start 139.93125 81.76875) (end 138.4 83.3) (width 0.2) (layer "F.Cu") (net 11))
 (segment (start 107 85.3) (end 107 88.4) (width 0.2) (layer "F.Cu") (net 11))
 (segment (start 107.76 89.16) (end 110.89 89.16) (width 0.2) (layer "F.Cu") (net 11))
 (segment (start 152.635705 73.08875) (end 144.255947 81.468508) (width 0.2) (layer "F.Cu") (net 11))
 (segment (start 138.4 83.3) (end 109 83.3) (width 0.2) (layer "F.Cu") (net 11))
 (via (at 139.93125 81.76875) (size 0.6) (drill 0.3) (layers "F.Cu" "B.Cu") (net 11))
 (via (at 144.255947 81.468508) (size 0.6) (drill 0.3) (layers "F.Cu" "B.Cu") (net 11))
 (segment (start 141.53125 83.36875) (end 142.355705 83.36875) (width 0.2) (layer "B.Cu") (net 11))
 (segment (start 139.93125 81.76875) (end 141.53125 83.36875) (width 0.2) (layer "B.Cu") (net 11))
 (segment (start 142.355705 83.36875) (end 144.255947 81.468508) (width 0.2) (layer "B.Cu") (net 11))
 (segment (start 154.05125 70.54875) (end 159.79625 70.54875) (width 0.2) (layer "F.Cu") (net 10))
 (segment (start 140.023265 84.276735) (end 139.8 84.5) (width 0.2) (layer "F.Cu") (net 10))
 (segment (start 139.8 84.5) (end 139.51857 84.5) (width 0.2) (layer "F.Cu") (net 10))
 (segment (start 139.51757 84.501) (end 126.2661 84.501) (width 0.2) (layer "F.Cu") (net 10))
 (segment (start 126.2661 84.501) (end 125.8 84.9671) (width 0.2) (layer "F.Cu") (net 10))
 (segment (start 140.376735 83.924678) (end 140.024678 84.276735) (width 0.2) (layer "F.Cu") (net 10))
 (segment (start 139.51857 84.5) (end 139.51757 84.501) (width 0.2) (layer "F.Cu") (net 10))
 (segment (start 143.53125 80.96875) (end 143.63125 80.96875) (width 0.2) (layer "F.Cu") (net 10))
 (segment (start 143.63125 80.96875) (end 154.05125 70.54875) (width 0.2) (layer "F.Cu") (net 10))
 (segment (start 140.024678 84.276735) (end 140.023265 84.276735) (width 0.2) (layer "F.Cu") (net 10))
 (segment (start 142.03125 82.26875) (end 140.376735 83.923265) (width 0.2) (layer "F.Cu") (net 10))
 (segment (start 142.33125 82.16875) (end 142.23125 82.26875) (width 0.2) (layer "F.Cu") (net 10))
 (segment (start 126.36 89.16) (end 129.94 89.16) (width 0.2) (layer "F.Cu") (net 10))
 (segment (start 125.8 84.9671) (end 125.8 88.6) (width 0.2) (layer "F.Cu") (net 10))
 (segment (start 140.376735 83.923265) (end 140.376735 83.924678) (width 0.2) (layer "F.Cu") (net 10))
 (segment (start 142.23125 82.26875) (end 142.03125 82.26875) (width 0.2) (layer "F.Cu") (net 10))
 (segment (start 125.8 88.6) (end 126.36 89.16) (width 0.2) (layer "F.Cu") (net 10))
 (via (at 142.33125 82.16875) (size 0.6) (drill 0.3) (layers "F.Cu" "B.Cu") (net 10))
 (via (at 143.53125 80.96875) (size 0.6) (drill 0.3) (layers "F.Cu" "B.Cu") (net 10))
 (segment (start 142.33125 82.16875) (end 143.53125 80.96875) (width 0.2) (layer "B.Cu") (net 10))
 (segment (start 148.99 89.16) (end 146.76 89.16) (width 0.2) (layer "F.Cu") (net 8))
 (segment (start 145.4 84.5) (end 146.9 83) (width 0.2) (layer "F.Cu") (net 8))
 (segment (start 145.4 87.8) (end 145.4 84.5) (width 0.2) (layer "F.Cu") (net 8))
 (segment (start 146.76 89.16) (end 145.4 87.8) (width 0.2) (layer "F.Cu") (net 8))
 (segment (start 146.9 83) (end 147.4 83) (width 0.2) (layer "F.Cu") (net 8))
 (via (at 147.4 83) (size 0.6) (drill 0.3) (layers "F.Cu" "B.Cu") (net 8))
 (segment (start 147.4 83) (end 144.55625 80.15625) (width 0.2) (layer "B.Cu") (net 8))
 (segment (start 144.55625 80.15625) (end 144.55625 78.16875) (width 0.2) (layer "B.Cu") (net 8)))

